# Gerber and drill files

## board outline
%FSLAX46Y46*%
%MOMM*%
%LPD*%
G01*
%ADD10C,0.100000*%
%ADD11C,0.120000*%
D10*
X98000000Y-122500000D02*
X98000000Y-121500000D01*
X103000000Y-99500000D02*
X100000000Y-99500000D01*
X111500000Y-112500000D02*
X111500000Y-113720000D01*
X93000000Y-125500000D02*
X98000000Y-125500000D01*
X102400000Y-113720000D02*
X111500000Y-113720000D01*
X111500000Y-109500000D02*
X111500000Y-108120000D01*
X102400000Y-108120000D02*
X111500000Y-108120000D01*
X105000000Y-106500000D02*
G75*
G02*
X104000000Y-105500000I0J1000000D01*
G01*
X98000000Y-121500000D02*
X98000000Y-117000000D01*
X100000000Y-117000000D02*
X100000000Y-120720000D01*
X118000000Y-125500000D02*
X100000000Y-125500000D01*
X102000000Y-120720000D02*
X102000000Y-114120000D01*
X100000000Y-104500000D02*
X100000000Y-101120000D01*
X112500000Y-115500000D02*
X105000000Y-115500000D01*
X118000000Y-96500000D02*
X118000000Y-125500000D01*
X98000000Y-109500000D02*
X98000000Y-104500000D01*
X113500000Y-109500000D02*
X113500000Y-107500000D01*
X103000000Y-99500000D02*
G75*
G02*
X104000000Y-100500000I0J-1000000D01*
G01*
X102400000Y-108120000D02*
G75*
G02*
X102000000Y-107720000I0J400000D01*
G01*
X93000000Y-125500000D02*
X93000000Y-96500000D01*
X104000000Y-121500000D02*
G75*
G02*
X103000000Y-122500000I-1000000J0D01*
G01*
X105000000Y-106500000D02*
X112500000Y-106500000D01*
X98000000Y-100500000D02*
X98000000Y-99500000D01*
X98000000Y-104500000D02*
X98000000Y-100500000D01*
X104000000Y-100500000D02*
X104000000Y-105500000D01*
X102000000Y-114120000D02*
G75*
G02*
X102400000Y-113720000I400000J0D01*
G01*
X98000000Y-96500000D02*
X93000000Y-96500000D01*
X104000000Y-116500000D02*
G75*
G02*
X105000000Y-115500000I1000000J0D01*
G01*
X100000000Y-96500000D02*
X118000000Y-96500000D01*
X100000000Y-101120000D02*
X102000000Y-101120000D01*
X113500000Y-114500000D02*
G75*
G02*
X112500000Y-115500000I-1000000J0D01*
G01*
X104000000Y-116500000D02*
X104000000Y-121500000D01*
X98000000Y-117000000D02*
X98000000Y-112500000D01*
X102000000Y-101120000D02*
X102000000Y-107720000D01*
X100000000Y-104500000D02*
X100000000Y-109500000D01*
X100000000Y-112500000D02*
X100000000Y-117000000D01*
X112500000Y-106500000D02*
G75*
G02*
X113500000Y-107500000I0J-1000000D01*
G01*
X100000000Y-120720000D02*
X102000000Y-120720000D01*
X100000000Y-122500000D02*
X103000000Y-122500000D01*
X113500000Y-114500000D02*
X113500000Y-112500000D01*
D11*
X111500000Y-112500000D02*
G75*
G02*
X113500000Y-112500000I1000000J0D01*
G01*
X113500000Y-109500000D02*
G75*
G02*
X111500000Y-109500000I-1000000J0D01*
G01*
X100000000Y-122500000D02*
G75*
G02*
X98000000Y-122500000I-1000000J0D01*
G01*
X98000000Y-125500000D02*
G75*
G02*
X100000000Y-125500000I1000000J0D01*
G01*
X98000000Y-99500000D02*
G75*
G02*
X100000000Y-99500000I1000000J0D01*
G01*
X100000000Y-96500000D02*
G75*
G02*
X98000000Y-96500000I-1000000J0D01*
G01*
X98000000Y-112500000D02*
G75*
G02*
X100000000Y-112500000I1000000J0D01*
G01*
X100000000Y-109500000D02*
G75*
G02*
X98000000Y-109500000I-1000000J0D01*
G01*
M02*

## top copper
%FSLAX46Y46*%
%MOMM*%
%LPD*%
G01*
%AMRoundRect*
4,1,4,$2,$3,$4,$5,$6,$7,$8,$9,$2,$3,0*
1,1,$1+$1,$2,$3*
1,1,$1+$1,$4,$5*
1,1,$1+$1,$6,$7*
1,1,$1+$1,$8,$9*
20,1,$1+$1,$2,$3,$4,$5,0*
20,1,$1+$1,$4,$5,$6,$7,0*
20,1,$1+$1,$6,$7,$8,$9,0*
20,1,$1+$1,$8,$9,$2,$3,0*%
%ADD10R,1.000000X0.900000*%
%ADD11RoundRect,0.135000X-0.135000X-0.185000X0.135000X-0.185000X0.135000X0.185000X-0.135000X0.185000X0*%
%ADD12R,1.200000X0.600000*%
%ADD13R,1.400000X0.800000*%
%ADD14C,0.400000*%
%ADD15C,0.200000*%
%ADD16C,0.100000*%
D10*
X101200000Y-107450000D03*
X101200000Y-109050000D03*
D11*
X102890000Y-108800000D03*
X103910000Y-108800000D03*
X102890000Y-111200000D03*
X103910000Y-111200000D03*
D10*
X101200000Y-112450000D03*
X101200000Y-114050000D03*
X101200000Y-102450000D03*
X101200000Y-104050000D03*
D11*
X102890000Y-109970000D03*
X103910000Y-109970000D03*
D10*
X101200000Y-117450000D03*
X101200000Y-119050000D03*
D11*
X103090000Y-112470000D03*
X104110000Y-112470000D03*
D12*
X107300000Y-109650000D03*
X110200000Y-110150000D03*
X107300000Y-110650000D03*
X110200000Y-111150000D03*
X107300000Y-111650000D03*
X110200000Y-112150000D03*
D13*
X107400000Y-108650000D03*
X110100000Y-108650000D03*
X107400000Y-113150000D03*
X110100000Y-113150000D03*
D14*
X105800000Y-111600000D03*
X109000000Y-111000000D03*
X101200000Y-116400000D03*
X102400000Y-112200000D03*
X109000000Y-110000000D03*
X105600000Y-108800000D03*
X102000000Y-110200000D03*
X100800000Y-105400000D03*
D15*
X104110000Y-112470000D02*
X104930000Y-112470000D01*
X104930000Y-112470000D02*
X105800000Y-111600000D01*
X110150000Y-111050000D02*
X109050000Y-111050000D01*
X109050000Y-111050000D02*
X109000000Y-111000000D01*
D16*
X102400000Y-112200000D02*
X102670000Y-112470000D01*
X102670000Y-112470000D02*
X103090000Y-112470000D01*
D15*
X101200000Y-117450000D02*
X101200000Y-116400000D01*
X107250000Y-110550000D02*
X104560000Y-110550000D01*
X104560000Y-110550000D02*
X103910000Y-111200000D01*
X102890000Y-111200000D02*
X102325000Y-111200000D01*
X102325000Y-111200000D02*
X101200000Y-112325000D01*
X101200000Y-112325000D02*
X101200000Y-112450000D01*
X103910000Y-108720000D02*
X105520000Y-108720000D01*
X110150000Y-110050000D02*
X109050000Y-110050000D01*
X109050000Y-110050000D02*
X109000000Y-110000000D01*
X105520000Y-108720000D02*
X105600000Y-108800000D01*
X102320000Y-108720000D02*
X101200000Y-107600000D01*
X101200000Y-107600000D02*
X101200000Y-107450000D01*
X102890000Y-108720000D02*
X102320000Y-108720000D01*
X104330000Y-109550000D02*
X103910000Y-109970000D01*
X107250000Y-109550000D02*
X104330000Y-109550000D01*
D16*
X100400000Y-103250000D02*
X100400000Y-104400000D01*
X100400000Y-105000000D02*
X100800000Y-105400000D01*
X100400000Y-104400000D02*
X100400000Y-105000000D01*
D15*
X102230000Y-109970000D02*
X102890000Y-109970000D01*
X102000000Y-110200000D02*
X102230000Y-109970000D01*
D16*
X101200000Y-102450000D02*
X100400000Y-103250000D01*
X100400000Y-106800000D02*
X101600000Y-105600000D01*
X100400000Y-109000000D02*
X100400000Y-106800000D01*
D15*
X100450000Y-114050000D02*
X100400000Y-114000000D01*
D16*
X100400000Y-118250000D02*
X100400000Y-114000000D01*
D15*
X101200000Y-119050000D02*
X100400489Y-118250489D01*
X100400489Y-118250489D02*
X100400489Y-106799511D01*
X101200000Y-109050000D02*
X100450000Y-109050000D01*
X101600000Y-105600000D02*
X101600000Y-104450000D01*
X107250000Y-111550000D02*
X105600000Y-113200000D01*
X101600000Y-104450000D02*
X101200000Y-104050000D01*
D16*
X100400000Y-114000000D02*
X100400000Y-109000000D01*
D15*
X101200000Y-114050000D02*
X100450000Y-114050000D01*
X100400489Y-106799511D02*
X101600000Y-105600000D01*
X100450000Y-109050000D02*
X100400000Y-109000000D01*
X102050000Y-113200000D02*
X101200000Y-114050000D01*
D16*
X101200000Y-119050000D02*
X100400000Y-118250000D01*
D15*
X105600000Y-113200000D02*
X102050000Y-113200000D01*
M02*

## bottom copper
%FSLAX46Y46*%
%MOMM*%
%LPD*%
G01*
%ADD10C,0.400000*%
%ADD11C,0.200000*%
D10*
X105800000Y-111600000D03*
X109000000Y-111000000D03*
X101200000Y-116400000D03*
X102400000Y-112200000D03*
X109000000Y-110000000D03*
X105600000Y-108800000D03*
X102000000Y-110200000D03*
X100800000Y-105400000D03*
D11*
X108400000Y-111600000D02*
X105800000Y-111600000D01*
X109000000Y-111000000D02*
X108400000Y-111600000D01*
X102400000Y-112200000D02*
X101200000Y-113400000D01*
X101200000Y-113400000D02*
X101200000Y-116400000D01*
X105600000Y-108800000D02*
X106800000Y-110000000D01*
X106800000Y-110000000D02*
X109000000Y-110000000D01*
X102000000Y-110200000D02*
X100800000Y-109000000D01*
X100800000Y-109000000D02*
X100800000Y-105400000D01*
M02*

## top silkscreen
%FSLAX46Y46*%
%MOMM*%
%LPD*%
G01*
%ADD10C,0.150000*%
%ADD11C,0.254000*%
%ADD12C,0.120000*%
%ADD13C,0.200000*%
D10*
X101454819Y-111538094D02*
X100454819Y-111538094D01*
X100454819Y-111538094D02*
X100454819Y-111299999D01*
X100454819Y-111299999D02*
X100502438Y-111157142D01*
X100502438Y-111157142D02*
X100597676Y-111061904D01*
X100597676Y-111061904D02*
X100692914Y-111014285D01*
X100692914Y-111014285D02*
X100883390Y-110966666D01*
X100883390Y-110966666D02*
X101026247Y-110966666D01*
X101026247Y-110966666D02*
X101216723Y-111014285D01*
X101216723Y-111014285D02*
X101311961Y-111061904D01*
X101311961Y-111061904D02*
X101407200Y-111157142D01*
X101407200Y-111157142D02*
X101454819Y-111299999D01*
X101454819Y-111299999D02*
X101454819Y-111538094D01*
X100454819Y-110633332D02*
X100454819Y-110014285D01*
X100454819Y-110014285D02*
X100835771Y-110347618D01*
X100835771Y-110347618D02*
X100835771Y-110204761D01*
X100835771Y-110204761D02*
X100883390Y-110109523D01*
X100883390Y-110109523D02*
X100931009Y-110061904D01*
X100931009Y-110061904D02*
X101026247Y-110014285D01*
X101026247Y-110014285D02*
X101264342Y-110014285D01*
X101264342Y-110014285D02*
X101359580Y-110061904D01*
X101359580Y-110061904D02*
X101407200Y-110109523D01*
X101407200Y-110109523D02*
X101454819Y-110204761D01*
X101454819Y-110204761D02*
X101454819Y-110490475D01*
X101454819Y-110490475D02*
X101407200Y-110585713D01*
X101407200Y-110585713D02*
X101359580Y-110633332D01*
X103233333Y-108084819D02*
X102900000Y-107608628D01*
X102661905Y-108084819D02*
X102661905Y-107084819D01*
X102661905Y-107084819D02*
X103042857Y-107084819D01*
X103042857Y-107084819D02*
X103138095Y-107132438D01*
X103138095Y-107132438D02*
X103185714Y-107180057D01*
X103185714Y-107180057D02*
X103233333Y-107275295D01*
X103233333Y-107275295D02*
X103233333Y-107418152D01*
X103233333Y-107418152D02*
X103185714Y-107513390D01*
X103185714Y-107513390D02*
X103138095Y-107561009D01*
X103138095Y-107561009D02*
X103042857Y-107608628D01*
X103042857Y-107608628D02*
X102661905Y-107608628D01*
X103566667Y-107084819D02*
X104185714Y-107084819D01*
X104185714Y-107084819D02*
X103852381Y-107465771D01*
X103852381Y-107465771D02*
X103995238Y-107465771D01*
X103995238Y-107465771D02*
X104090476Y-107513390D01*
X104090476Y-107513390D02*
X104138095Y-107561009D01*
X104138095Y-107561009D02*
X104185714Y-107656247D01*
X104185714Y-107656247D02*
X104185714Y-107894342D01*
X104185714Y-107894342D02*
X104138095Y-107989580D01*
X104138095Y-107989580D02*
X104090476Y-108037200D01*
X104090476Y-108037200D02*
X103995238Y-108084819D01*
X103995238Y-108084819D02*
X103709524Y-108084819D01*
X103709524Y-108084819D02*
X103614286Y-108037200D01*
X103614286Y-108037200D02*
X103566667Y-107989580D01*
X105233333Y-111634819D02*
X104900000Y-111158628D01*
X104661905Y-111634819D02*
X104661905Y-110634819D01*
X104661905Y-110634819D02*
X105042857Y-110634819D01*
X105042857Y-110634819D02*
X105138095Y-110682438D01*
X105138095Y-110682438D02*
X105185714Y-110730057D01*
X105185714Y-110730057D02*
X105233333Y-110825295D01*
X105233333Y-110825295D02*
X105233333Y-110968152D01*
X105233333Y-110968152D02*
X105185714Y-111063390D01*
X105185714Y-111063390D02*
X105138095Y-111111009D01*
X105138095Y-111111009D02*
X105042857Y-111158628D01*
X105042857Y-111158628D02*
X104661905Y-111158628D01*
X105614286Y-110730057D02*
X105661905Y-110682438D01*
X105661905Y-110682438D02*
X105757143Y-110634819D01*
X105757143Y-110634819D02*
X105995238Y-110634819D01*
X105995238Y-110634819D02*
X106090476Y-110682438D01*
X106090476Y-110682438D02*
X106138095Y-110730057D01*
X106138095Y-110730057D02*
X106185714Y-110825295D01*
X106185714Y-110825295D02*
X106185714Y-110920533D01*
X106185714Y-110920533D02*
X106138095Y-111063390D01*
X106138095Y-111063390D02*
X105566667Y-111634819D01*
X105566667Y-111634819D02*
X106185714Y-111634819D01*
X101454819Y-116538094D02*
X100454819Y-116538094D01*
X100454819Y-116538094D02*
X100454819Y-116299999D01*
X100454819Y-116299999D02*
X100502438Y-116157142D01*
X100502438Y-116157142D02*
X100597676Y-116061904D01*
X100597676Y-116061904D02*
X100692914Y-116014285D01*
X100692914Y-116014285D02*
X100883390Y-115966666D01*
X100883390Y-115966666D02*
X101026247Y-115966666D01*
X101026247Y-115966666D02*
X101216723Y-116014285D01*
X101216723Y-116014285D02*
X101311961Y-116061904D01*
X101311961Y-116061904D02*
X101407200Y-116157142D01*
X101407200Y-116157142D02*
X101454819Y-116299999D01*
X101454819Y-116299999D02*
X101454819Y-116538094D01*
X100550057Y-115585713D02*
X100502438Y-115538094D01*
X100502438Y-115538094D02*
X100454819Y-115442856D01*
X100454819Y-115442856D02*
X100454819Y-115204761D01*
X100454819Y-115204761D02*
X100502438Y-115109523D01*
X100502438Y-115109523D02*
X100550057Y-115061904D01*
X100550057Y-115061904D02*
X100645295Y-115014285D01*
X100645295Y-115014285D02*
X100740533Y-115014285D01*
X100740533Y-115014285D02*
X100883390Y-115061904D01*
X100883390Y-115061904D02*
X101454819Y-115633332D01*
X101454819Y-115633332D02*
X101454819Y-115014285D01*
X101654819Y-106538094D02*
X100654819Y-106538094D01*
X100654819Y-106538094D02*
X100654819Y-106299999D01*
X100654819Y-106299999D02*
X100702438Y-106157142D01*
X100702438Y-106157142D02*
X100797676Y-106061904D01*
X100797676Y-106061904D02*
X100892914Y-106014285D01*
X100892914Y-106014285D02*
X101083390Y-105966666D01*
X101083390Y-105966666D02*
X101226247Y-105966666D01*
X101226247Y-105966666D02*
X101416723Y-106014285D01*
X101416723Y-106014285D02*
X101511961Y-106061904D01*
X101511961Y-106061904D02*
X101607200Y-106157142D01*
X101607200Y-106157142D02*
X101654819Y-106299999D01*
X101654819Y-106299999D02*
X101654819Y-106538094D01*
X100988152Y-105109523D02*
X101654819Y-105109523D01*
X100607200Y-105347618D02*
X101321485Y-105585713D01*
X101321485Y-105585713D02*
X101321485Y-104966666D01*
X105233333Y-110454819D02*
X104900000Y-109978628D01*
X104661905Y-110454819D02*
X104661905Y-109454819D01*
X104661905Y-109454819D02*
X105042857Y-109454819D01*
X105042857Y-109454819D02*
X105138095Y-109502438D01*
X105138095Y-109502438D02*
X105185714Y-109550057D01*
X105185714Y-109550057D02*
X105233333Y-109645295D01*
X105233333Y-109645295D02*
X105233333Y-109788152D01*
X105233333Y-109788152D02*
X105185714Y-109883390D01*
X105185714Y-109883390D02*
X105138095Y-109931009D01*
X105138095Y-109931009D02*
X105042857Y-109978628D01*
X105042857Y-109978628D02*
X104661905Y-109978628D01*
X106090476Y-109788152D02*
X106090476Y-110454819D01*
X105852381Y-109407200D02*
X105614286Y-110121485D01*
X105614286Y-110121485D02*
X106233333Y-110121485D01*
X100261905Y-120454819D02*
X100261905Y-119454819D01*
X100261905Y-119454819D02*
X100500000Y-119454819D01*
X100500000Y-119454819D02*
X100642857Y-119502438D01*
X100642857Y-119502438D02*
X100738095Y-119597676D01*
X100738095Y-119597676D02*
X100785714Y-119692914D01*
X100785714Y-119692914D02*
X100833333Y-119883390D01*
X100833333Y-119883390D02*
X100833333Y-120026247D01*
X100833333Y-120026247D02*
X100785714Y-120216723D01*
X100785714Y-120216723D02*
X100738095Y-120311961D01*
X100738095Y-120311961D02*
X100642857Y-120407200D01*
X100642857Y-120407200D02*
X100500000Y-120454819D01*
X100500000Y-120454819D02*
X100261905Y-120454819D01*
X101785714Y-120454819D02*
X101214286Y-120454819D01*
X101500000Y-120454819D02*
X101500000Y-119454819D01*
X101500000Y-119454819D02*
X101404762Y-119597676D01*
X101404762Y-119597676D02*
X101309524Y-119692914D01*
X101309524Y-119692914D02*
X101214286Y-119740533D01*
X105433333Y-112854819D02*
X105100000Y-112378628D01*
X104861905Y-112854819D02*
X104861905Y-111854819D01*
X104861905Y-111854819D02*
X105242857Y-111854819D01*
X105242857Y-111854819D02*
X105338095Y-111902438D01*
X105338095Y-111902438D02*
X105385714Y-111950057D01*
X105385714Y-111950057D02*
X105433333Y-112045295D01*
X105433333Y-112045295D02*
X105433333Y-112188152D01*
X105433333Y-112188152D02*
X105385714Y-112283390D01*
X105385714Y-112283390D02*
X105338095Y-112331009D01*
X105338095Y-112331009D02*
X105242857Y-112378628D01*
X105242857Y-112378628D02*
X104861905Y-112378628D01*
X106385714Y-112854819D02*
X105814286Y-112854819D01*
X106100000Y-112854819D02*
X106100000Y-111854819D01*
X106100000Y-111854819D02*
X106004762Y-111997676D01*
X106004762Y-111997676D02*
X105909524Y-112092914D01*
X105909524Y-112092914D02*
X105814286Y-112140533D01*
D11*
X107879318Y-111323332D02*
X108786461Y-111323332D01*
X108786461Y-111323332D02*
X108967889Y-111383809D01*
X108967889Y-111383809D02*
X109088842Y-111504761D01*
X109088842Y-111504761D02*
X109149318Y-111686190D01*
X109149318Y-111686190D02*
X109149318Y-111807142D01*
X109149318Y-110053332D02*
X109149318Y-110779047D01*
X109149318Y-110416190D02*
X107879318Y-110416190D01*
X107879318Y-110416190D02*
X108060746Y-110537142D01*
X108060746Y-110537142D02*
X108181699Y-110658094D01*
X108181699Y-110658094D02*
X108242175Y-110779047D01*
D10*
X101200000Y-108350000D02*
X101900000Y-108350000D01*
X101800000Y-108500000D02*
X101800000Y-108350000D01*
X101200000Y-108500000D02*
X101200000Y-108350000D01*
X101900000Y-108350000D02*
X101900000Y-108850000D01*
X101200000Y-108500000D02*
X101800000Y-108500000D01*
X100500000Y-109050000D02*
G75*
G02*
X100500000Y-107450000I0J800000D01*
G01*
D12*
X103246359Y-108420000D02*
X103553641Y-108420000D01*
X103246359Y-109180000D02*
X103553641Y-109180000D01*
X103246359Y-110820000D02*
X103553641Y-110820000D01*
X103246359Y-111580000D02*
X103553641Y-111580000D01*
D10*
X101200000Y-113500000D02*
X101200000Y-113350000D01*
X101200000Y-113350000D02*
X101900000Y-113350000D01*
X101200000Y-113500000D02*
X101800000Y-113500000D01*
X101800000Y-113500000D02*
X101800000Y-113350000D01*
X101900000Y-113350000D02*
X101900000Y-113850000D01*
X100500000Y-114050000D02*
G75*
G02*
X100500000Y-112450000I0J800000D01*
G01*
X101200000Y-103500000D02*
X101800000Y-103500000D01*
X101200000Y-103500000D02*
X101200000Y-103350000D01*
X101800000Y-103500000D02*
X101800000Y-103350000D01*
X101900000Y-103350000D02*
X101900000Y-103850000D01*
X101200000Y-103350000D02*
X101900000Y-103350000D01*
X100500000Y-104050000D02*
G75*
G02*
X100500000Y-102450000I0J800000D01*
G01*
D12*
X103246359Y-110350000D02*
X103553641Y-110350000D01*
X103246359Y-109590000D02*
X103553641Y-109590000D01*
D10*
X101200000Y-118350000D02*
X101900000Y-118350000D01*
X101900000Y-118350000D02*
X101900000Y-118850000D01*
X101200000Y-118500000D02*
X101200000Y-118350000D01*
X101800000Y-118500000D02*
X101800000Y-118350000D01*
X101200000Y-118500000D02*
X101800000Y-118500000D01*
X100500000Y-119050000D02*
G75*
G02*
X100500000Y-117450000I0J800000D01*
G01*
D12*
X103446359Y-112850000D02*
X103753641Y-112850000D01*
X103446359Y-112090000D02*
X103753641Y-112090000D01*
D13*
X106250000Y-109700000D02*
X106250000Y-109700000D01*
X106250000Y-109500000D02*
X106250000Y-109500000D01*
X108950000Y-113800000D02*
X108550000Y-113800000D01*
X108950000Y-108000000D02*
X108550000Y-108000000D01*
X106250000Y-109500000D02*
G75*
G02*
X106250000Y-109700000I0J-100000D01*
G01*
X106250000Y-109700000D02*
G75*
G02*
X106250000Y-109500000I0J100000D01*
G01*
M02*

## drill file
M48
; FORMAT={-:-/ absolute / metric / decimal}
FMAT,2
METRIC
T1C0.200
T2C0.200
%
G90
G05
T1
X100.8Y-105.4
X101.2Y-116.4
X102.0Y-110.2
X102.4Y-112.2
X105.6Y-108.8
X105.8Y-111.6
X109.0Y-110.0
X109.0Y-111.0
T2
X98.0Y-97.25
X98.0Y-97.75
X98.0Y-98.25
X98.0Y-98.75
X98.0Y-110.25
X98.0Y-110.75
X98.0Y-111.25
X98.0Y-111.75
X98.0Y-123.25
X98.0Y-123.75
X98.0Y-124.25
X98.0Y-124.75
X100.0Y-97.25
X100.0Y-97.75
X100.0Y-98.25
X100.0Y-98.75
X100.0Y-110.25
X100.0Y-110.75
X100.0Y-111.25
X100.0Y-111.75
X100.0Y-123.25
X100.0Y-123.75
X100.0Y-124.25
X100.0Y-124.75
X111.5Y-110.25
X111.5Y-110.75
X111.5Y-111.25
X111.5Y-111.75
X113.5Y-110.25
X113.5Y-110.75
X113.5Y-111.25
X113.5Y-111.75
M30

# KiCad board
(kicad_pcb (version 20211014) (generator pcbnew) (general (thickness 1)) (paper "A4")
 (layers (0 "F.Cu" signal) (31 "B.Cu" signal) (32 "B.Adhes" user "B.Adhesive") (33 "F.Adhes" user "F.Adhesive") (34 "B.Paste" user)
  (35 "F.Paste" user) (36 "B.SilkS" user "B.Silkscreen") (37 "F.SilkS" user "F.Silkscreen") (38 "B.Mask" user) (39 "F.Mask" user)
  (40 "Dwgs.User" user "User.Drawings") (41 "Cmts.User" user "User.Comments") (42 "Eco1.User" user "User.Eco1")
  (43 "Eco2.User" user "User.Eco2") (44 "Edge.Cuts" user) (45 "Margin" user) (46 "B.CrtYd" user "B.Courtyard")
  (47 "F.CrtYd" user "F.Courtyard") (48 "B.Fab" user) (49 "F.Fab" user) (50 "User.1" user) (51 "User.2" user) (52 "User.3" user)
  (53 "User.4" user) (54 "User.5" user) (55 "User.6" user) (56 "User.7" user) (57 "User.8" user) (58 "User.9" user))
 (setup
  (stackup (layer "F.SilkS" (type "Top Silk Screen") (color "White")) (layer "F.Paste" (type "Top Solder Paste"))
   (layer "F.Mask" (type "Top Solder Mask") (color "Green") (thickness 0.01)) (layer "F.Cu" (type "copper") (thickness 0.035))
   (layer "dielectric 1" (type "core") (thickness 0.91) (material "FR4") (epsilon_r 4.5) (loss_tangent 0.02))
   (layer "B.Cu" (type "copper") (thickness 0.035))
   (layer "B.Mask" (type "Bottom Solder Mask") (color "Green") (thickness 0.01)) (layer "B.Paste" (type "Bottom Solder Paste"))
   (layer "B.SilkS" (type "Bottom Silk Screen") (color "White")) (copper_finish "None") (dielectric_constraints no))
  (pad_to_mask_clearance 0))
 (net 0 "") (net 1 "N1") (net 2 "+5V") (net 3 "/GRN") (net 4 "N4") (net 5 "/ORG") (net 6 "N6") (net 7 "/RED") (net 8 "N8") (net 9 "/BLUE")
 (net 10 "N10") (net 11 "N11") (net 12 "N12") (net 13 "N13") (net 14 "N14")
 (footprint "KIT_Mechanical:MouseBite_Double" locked (layer "F.Cu") (at 112.5 111) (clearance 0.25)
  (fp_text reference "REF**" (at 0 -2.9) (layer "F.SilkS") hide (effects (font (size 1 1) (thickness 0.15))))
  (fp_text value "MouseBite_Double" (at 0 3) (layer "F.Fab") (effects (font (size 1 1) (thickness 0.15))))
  (fp_arc (start -1 1.5) (mid 0 0.5) (end 1 1.5) (layer "Edge.Cuts") (width 0.12))
  (fp_arc (start 1 -1.5) (mid 0 -0.5) (end -1 -1.5) (layer "Edge.Cuts") (width 0.12))
  (pad "" np_thru_hole circle locked (at -1 0.75) (size 0.2 0.2) (drill 0.2) (layers *.Cu *.Mask))
  (pad "" np_thru_hole circle locked (at -1 0.25) (size 0.2 0.2) (drill 0.2) (layers *.Cu *.Mask))
  (pad "" np_thru_hole circle locked (at -1 -0.25) (size 0.2 0.2) (drill 0.2) (layers *.Cu *.Mask))
  (pad "" np_thru_hole circle locked (at -1 -0.75) (size 0.2 0.2) (drill 0.2) (layers *.Cu *.Mask))
  (pad "" np_thru_hole circle locked (at 1 0.75 180) (size 0.2 0.2) (drill 0.2) (layers *.Cu *.Mask))
  (pad "" np_thru_hole circle locked (at 1 -0.25 180) (size 0.2 0.2) (drill 0.2) (layers *.Cu *.Mask))
  (pad "" np_thru_hole circle locked (at 1 0.25 180) (size 0.2 0.2) (drill 0.2) (layers *.Cu *.Mask))
  (pad "" np_thru_hole circle locked (at 1 -0.75 180) (size 0.2 0.2) (drill 0.2) (layers *.Cu *.Mask)))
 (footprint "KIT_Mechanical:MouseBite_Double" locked (layer "F.Cu") (at 99 124) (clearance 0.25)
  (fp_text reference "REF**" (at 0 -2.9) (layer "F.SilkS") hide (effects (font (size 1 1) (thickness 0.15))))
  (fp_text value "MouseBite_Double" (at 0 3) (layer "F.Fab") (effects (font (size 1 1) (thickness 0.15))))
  (fp_arc (start 1 -1.5) (mid 0 -0.5) (end -1 -1.5) (layer "Edge.Cuts") (width 0.12))
  (fp_arc (start -1 1.5) (mid 0 0.5) (end 1 1.5) (layer "Edge.Cuts") (width 0.12))
  (pad "" np_thru_hole circle locked (at -1 -0.75) (size 0.2 0.2) (drill 0.2) (layers *.Cu *.Mask))
  (pad "" np_thru_hole circle locked (at -1 0.25) (size 0.2 0.2) (drill 0.2) (layers *.Cu *.Mask))
  (pad "" np_thru_hole circle locked (at 1 0.25 180) (size 0.2 0.2) (drill 0.2) (layers *.Cu *.Mask))
  (pad "" np_thru_hole circle locked (at 1 -0.75 180) (size 0.2 0.2) (drill 0.2) (layers *.Cu *.Mask))
  (pad "" np_thru_hole circle locked (at -1 -0.25) (size 0.2 0.2) (drill 0.2) (layers *.Cu *.Mask))
  (pad "" np_thru_hole circle locked (at -1 0.75) (size 0.2 0.2) (drill 0.2) (layers *.Cu *.Mask))
  (pad "" np_thru_hole circle locked (at 1 0.75 180) (size 0.2 0.2) (drill 0.2) (layers *.Cu *.Mask))
  (pad "" np_thru_hole circle locked (at 1 -0.25 180) (size 0.2 0.2) (drill 0.2) (layers *.Cu *.Mask)))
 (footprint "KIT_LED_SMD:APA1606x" (layer "F.Cu") (at 101.2 108.25 -90)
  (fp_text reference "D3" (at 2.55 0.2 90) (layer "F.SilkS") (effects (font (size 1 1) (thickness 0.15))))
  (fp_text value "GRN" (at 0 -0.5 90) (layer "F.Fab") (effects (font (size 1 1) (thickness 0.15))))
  (fp_line (start 0.1 0) (end 0.1 -0.7) (layer "F.SilkS") (width 0.15))
  (fp_line (start 0.25 -0.6) (end 0.1 -0.6) (layer "F.SilkS") (width 0.15))
  (fp_line (start 0.25 0) (end 0.1 0) (layer "F.SilkS") (width 0.15))
  (fp_line (start 0.1 -0.7) (end 0.6 -0.7) (layer "F.SilkS") (width 0.15))
  (fp_line (start 0.25 0) (end 0.25 -0.6) (layer "F.SilkS") (width 0.15))
  (fp_arc (start 0.8 0.7) (mid 0 1.5) (end -0.8 0.7) (layer "F.SilkS") (width 0.15))
  (pad "1" smd rect (at -0.8 0 270) (size 0.9 1) (layers "F.Cu" "F.Paste" "F.Mask") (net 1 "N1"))
  (pad "2" smd rect (at 0.8 0 270) (size 0.9 1) (layers "F.Cu" "F.Paste" "F.Mask") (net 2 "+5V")))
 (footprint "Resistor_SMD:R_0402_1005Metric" (layer "F.Cu") (at 103.4 108.8)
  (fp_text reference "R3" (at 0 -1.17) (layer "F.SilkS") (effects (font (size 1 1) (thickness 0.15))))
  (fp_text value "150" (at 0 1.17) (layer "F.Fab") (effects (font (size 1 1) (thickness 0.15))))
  (fp_line (start -0.153641 -0.38) (end 0.153641 -0.38) (layer "F.SilkS") (width 0.12))
  (fp_line (start -0.153641 0.38) (end 0.153641 0.38) (layer "F.SilkS") (width 0.12))
  (pad "1" smd roundrect (at -0.51 0) (size 0.54 0.64) (layers "F.Cu" "F.Paste" "F.Mask") (roundrect_rratio 0.25) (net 1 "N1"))
  (pad "2" smd roundrect (at 0.51 0) (size 0.54 0.64) (layers "F.Cu" "F.Paste" "F.Mask") (roundrect_rratio 0.25) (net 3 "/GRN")))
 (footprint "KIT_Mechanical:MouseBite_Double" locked (layer "F.Cu") (at 99 98) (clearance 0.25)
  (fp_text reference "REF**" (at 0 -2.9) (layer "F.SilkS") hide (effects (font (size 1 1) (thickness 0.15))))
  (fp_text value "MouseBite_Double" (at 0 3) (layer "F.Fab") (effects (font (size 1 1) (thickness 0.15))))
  (fp_arc (start -1 1.5) (mid 0 0.5) (end 1 1.5) (layer "Edge.Cuts") (width 0.12))
  (fp_arc (start 1 -1.5) (mid 0 -0.5) (end -1 -1.5) (layer "Edge.Cuts") (width 0.12))
  (pad "" np_thru_hole circle locked (at 1 -0.75 180) (size 0.2 0.2) (drill 0.2) (layers *.Cu *.Mask))
  (pad "" np_thru_hole circle locked (at -1 -0.75) (size 0.2 0.2) (drill 0.2) (layers *.Cu *.Mask))
  (pad "" np_thru_hole circle locked (at 1 -0.25 180) (size 0.2 0.2) (drill 0.2) (layers *.Cu *.Mask))
  (pad "" np_thru_hole circle locked (at -1 0.25) (size 0.2 0.2) (drill 0.2) (layers *.Cu *.Mask))
  (pad "" np_thru_hole circle locked (at 1 0.25 180) (size 0.2 0.2) (drill 0.2) (layers *.Cu *.Mask))
  (pad "" np_thru_hole circle locked (at -1 0.75) (size 0.2 0.2) (drill 0.2) (layers *.Cu *.Mask))
  (pad "" np_thru_hole circle locked (at -1 -0.25) (size 0.2 0.2) (drill 0.2) (layers *.Cu *.Mask))
  (pad "" np_thru_hole circle locked (at 1 0.75 180) (size 0.2 0.2) (drill 0.2) (layers *.Cu *.Mask)))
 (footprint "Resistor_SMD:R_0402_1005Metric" (layer "F.Cu") (at 103.4 111.2)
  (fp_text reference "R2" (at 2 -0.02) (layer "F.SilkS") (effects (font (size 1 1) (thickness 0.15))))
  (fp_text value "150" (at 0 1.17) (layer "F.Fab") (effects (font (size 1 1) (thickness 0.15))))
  (fp_line (start -0.153641 -0.38) (end 0.153641 -0.38) (layer "F.SilkS") (width 0.12))
  (fp_line (start -0.153641 0.38) (end 0.153641 0.38) (layer "F.SilkS") (width 0.12))
  (pad "1" smd roundrect (at -0.51 0) (size 0.54 0.64) (layers "F.Cu" "F.Paste" "F.Mask") (roundrect_rratio 0.25) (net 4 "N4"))
  (pad "2" smd roundrect (at 0.51 0) (size 0.54 0.64) (layers "F.Cu" "F.Paste" "F.Mask") (roundrect_rratio 0.25) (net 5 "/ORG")))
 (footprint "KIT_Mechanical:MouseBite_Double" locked (layer "F.Cu") (at 99 111) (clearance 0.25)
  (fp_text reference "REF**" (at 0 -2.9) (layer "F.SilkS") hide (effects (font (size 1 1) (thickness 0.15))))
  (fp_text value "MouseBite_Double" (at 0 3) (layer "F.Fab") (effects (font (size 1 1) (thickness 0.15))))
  (fp_arc (start -1 1.5) (mid 0 0.5) (end 1 1.5) (layer "Edge.Cuts") (width 0.12))
  (fp_arc (start 1 -1.5) (mid 0 -0.5) (end -1 -1.5) (layer "Edge.Cuts") (width 0.12))
  (pad "" np_thru_hole circle locked (at -1 -0.25) (size 0.2 0.2) (drill 0.2) (layers *.Cu *.Mask))
  (pad "" np_thru_hole circle locked (at -1 -0.75) (size 0.2 0.2) (drill 0.2) (layers *.Cu *.Mask))
  (pad "" np_thru_hole circle locked (at -1 0.25) (size 0.2 0.2) (drill 0.2) (layers *.Cu *.Mask))
  (pad "" np_thru_hole circle locked (at 1 0.25 180) (size 0.2 0.2) (drill 0.2) (layers *.Cu *.Mask))
  (pad "" np_thru_hole circle locked (at 1 -0.75 180) (size 0.2 0.2) (drill 0.2) (layers *.Cu *.Mask))
  (pad "" np_thru_hole circle locked (at 1 0.75 180) (size 0.2 0.2) (drill 0.2) (layers *.Cu *.Mask))
  (pad "" np_thru_hole circle locked (at 1 -0.25 180) (size 0.2 0.2) (drill 0.2) (layers *.Cu *.Mask))
  (pad "" np_thru_hole circle locked (at -1 0.75) (size 0.2 0.2) (drill 0.2) (layers *.Cu *.Mask)))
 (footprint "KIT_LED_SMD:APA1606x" (layer "F.Cu") (at 101.2 113.25 -90)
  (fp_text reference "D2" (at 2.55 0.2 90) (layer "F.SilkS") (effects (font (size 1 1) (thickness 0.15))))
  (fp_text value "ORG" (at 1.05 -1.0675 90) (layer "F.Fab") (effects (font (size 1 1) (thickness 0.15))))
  (fp_line (start 0.25 0) (end 0.1 0) (layer "F.SilkS") (width 0.15))
  (fp_line (start 0.1 0) (end 0.1 -0.7) (layer "F.SilkS") (width 0.15))
  (fp_line (start 0.25 0) (end 0.25 -0.6) (layer "F.SilkS") (width 0.15))
  (fp_line (start 0.25 -0.6) (end 0.1 -0.6) (layer "F.SilkS") (width 0.15))
  (fp_line (start 0.1 -0.7) (end 0.6 -0.7) (layer "F.SilkS") (width 0.15))
  (fp_arc (start 0.8 0.7) (mid 0 1.5) (end -0.8 0.7) (layer "F.SilkS") (width 0.15))
  (pad "1" smd rect (at -0.8 0 270) (size 0.9 1) (layers "F.Cu" "F.Paste" "F.Mask") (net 4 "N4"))
  (pad "2" smd rect (at 0.8 0 270) (size 0.9 1) (layers "F.Cu" "F.Paste" "F.Mask") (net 2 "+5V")))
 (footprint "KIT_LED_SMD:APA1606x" (layer "F.Cu") (at 101.2 103.25 -90)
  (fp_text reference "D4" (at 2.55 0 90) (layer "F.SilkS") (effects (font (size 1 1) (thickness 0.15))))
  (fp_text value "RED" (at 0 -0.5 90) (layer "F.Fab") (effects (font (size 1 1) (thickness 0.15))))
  (fp_line (start 0.25 0) (end 0.25 -0.6) (layer "F.SilkS") (width 0.15))
  (fp_line (start 0.25 0) (end 0.1 0) (layer "F.SilkS") (width 0.15))
  (fp_line (start 0.25 -0.6) (end 0.1 -0.6) (layer "F.SilkS") (width 0.15))
  (fp_line (start 0.1 -0.7) (end 0.6 -0.7) (layer "F.SilkS") (width 0.15))
  (fp_line (start 0.1 0) (end 0.1 -0.7) (layer "F.SilkS") (width 0.15))
  (fp_arc (start 0.8 0.7) (mid 0 1.5) (end -0.8 0.7) (layer "F.SilkS") (width 0.15))
  (pad "1" smd rect (at -0.8 0 270) (size 0.9 1) (layers "F.Cu" "F.Paste" "F.Mask") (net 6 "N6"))
  (pad "2" smd rect (at 0.8 0 270) (size 0.9 1) (layers "F.Cu" "F.Paste" "F.Mask") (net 2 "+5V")))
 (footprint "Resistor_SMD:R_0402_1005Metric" (layer "F.Cu") (at 103.4 109.97)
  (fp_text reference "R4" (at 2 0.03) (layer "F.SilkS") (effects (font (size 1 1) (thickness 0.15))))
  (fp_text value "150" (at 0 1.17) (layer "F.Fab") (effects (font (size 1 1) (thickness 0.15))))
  (fp_line (start -0.153641 0.38) (end 0.153641 0.38) (layer "F.SilkS") (width 0.12))
  (fp_line (start -0.153641 -0.38) (end 0.153641 -0.38) (layer "F.SilkS") (width 0.12))
  (pad "1" smd roundrect (at -0.51 0) (size 0.54 0.64) (layers "F.Cu" "F.Paste" "F.Mask") (roundrect_rratio 0.25) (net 6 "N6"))
  (pad "2" smd roundrect (at 0.51 0) (size 0.54 0.64) (layers "F.Cu" "F.Paste" "F.Mask") (roundrect_rratio 0.25) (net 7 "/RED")))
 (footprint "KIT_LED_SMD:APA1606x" (layer "F.Cu") (at 101.2 118.25 -90)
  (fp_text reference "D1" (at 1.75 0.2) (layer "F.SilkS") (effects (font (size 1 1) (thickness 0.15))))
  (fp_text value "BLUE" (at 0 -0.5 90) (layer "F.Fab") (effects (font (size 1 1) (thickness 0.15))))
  (fp_line (start 0.1 0) (end 0.1 -0.7) (layer "F.SilkS") (width 0.15))
  (fp_line (start 0.1 -0.7) (end 0.6 -0.7) (layer "F.SilkS") (width 0.15))
  (fp_line (start 0.25 0) (end 0.1 0) (layer "F.SilkS") (width 0.15))
  (fp_line (start 0.25 -0.6) (end 0.1 -0.6) (layer "F.SilkS") (width 0.15))
  (fp_line (start 0.25 0) (end 0.25 -0.6) (layer "F.SilkS") (width 0.15))
  (fp_arc (start 0.8 0.7) (mid 0 1.5) (end -0.8 0.7) (layer "F.SilkS") (width 0.15))
  (pad "1" smd rect (at -0.8 0 270) (size 0.9 1) (layers "F.Cu" "F.Paste" "F.Mask") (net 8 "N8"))
  (pad "2" smd rect (at 0.8 0 270) (size 0.9 1) (layers "F.Cu" "F.Paste" "F.Mask") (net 2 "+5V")))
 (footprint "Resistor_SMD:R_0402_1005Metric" (layer "F.Cu") (at 103.6 112.47)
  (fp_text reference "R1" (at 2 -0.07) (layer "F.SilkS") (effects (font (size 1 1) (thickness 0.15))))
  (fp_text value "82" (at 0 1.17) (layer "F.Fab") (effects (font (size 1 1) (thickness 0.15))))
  (fp_line (start -0.153641 0.38) (end 0.153641 0.38) (layer "F.SilkS") (width 0.12))
  (fp_line (start -0.153641 -0.38) (end 0.153641 -0.38) (layer "F.SilkS") (width 0.12))
  (pad "1" smd roundrect (at -0.51 0) (size 0.54 0.64) (layers "F.Cu" "F.Paste" "F.Mask") (roundrect_rratio 0.25) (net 8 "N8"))
  (pad "2" smd roundrect (at 0.51 0) (size 0.54 0.64) (layers "F.Cu" "F.Paste" "F.Mask") (roundrect_rratio 0.25) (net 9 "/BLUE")))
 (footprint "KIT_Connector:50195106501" (layer "F.Cu") (at 108.75 110.9 -90)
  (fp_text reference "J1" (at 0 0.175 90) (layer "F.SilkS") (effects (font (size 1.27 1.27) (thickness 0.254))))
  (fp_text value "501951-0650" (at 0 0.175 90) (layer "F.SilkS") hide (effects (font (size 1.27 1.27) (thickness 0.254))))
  (fp_line (start -1.2 2.5) (end -1.2 2.5) (layer "F.SilkS") (width 0.2))
  (fp_line (start -1.4 2.5) (end -1.4 2.5) (layer "F.SilkS") (width 0.2))
  (fp_line (start 2.9 -0.2) (end 2.9 0.2) (layer "F.SilkS") (width 0.2))
  (fp_line (start -2.9 -0.2) (end -2.9 0.2) (layer "F.SilkS") (width 0.2))
  (fp_arc (start -1.4 2.5) (mid -1.3 2.4) (end -1.2 2.5) (layer "F.SilkS") (width 0.2))
  (fp_arc (start -1.2 2.5) (mid -1.3 2.6) (end -1.4 2.5) (layer "F.SilkS") (width 0.2))
  (pad "1" smd rect (at -1.25 1.45 270) (size 0.6 1.2) (layers "F.Cu" "F.Paste" "F.Mask") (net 7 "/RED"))
  (pad "2" smd rect (at -0.75 -1.45 270) (size 0.6 1.2) (layers "F.Cu" "F.Paste" "F.Mask") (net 3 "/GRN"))
  (pad "3" smd rect (at -0.25 1.45 270) (size 0.6 1.2) (layers "F.Cu" "F.Paste" "F.Mask") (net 5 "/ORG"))
  (pad "4" smd rect (at 0.25 -1.45 270) (size 0.6 1.2) (layers "F.Cu" "F.Paste" "F.Mask") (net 9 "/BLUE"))
  (pad "5" smd rect (at 0.75 1.45 270) (size 0.6 1.2) (layers "F.Cu" "F.Paste" "F.Mask") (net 2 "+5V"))
  (pad "6" smd rect (at 1.25 -1.45 270) (size 0.6 1.2) (layers "F.Cu" "F.Paste" "F.Mask") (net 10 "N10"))
  (pad "MP1" smd rect (at -2.25 1.35 270) (size 0.8 1.4) (layers "F.Cu" "F.Paste" "F.Mask") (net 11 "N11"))
  (pad "MP2" smd rect (at -2.25 -1.35 270) (size 0.8 1.4) (layers "F.Cu" "F.Paste" "F.Mask") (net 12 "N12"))
  (pad "MP3" smd rect (at 2.25 1.35 270) (size 0.8 1.4) (layers "F.Cu" "F.Paste" "F.Mask") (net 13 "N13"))
  (pad "MP4" smd rect (at 2.25 -1.35 270) (size 0.8 1.4) (layers "F.Cu" "F.Paste" "F.Mask") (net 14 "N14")))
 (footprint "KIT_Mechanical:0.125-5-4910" (layer "B.Cu") (at 110.7 112.52 180)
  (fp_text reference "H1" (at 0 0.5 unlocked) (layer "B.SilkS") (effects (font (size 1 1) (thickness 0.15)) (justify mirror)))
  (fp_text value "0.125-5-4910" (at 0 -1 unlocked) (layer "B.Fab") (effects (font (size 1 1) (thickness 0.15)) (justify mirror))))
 (gr_line (start 98 122.5) (end 98 121.5) (layer "Edge.Cuts") (width 0.1))
 (gr_line (start 103 99.5) (end 100 99.5) (layer "Edge.Cuts") (width 0.1))
 (gr_line (start 111.5 112.5) (end 111.5 113.72) (layer "Edge.Cuts") (width 0.1))
 (gr_line (start 93 125.5) (end 98 125.5) (layer "Edge.Cuts") (width 0.1))
 (gr_line (start 102.4 113.72) (end 111.5 113.72) (layer "Edge.Cuts") (width 0.1))
 (gr_line (start 111.5 109.5) (end 111.5 108.12) (layer "Edge.Cuts") (width 0.1))
 (gr_line (start 102.4 108.12) (end 111.5 108.12) (layer "Edge.Cuts") (width 0.1))
 (gr_arc (start 105 106.5) (mid 104.292893 106.207107) (end 104 105.5) (layer "Edge.Cuts") (width 0.1))
 (gr_line (start 98 121.5) (end 98 117) (layer "Edge.Cuts") (width 0.1))
 (gr_line (start 100 117) (end 100 120.72) (layer "Edge.Cuts") (width 0.1))
 (gr_line (start 118 125.5) (end 100 125.5) (layer "Edge.Cuts") (width 0.1))
 (gr_line (start 102 120.72) (end 102 114.12) (layer "Edge.Cuts") (width 0.1))
 (gr_line (start 100 104.5) (end 100 101.12) (layer "Edge.Cuts") (width 0.1))
 (gr_line (start 112.5 115.5) (end 105 115.5) (layer "Edge.Cuts") (width 0.1))
 (gr_line (start 118 96.5) (end 118 125.5) (layer "Edge.Cuts") (width 0.1))
 (gr_line (start 98 109.5) (end 98 104.5) (layer "Edge.Cuts") (width 0.1))
 (gr_line (start 113.5 109.5) (end 113.5 107.5) (layer "Edge.Cuts") (width 0.1))
 (gr_arc (start 103 99.5) (mid 103.707107 99.792893) (end 104 100.5) (layer "Edge.Cuts") (width 0.1))
 (gr_arc (start 102.4 108.12) (mid 102.117157 108.002843) (end 102 107.72) (layer "Edge.Cuts") (width 0.1))
 (gr_line (start 93 125.5) (end 93 96.5) (layer "Edge.Cuts") (width 0.1))
 (gr_arc (start 104 121.5) (mid 103.707107 122.207107) (end 103 122.5) (layer "Edge.Cuts") (width 0.1))
 (gr_line (start 105 106.5) (end 112.5 106.5) (layer "Edge.Cuts") (width 0.1))
 (gr_line (start 98 100.5) (end 98 99.5) (layer "Edge.Cuts") (width 0.1))
 (gr_line (start 98 104.5) (end 98 100.5) (layer "Edge.Cuts") (width 0.1))
 (gr_line (start 104 100.5) (end 104 105.5) (layer "Edge.Cuts") (width 0.1))
 (gr_arc (start 102 114.12) (mid 102.117157 113.837157) (end 102.4 113.72) (layer "Edge.Cuts") (width 0.1))
 (gr_line (start 98 96.5) (end 93 96.5) (layer "Edge.Cuts") (width 0.1))
 (gr_arc (start 104 116.5) (mid 104.292893 115.792893) (end 105 115.5) (layer "Edge.Cuts") (width 0.1))
 (gr_line (start 100 96.5) (end 118 96.5) (layer "Edge.Cuts") (width 0.1))
 (gr_line (start 100 101.12) (end 102 101.12) (layer "Edge.Cuts") (width 0.1))
 (gr_arc (start 113.5 114.5) (mid 113.207107 115.207107) (end 112.5 115.5) (layer "Edge.Cuts") (width 0.1))
 (gr_line (start 104 116.5) (end 104 121.5) (layer "Edge.Cuts") (width 0.1))
 (gr_line (start 98 117) (end 98 112.5) (layer "Edge.Cuts") (width 0.1))
 (gr_line (start 102 101.12) (end 102 107.72) (layer "Edge.Cuts") (width 0.1))
 (gr_line (start 100 104.5) (end 100 109.5) (layer "Edge.Cuts") (width 0.1))
 (gr_line (start 100 112.5) (end 100 117) (layer "Edge.Cuts") (width 0.1))
 (gr_arc (start 112.5 106.5) (mid 113.207107 106.792893) (end 113.5 107.5) (layer "Edge.Cuts") (width 0.1))
 (gr_line (start 100 120.72) (end 102 120.72) (layer "Edge.Cuts") (width 0.1))
 (gr_line (start 100 122.5) (end 103 122.5) (layer "Edge.Cuts") (width 0.1))
 (gr_line (start 113.5 114.5) (end 113.5 112.5) (layer "Edge.Cuts") (width 0.1))
 (segment (start 104.11 112.47) (end 104.93 112.47) (width 0.2) (layer "F.Cu") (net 9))
 (segment (start 104.93 112.47) (end 105.8 111.6) (width 0.2) (layer "F.Cu") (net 9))
 (segment (start 110.15 111.05) (end 109.05 111.05) (width 0.2) (layer "F.Cu") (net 9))
 (segment (start 109.05 111.05) (end 109 111) (width 0.2) (layer "F.Cu") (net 9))
 (via (at 105.8 111.6) (size 0.4) (drill 0.2) (layers "F.Cu" "B.Cu") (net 9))
 (via (at 109 111) (size 0.4) (drill 0.2) (layers "F.Cu" "B.Cu") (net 9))
 (segment (start 108.4 111.6) (end 105.8 111.6) (width 0.2) (layer "B.Cu") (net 9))
 (segment (start 109 111) (end 108.4 111.6) (width 0.2) (layer "B.Cu") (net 9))
 (segment (start 102.4 112.2) (end 102.67 112.47) (width 0.1) (layer "F.Cu") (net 8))
 (segment (start 102.67 112.47) (end 103.09 112.47) (width 0.1) (layer "F.Cu") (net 8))
 (segment (start 101.2 117.45) (end 101.2 116.4) (width 0.2) (layer "F.Cu") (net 8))
 (via (at 101.2 116.4) (size 0.4) (drill 0.2) (layers "F.Cu" "B.Cu") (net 8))
 (via (at 102.4 112.2) (size 0.4) (drill 0.2) (layers "F.Cu" "B.Cu") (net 8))
 (segment (start 102.4 112.2) (end 101.2 113.4) (width 0.2) (layer "B.Cu") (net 8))
 (segment (start 101.2 113.4) (end 101.2 116.4) (width 0.2) (layer "B.Cu") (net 8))
 (segment (start 107.25 110.55) (end 104.56 110.55) (width 0.2) (layer "F.Cu") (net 5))
 (segment (start 104.56 110.55) (end 103.91 111.2) (width 0.2) (layer "F.Cu") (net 5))
 (segment (start 102.89 111.2) (end 102.325 111.2) (width 0.2) (layer "F.Cu") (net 4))
 (segment (start 102.325 111.2) (end 101.2 112.325) (width 0.2) (layer "F.Cu") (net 4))
 (segment (start 101.2 112.325) (end 101.2 112.45) (width 0.2) (layer "F.Cu") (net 4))
 (segment (start 103.91 108.72) (end 105.52 108.72) (width 0.2) (layer "F.Cu") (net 3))
 (segment (start 110.15 110.05) (end 109.05 110.05) (width 0.2) (layer "F.Cu") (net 3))
 (segment (start 109.05 110.05) (end 109 110) (width 0.2) (layer "F.Cu") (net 3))
 (segment (start 105.52 108.72) (end 105.6 108.8) (width 0.2) (layer "F.Cu") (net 3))
 (via (at 109 110) (size 0.4) (drill 0.2) (layers "F.Cu" "B.Cu") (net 3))
 (via (at 105.6 108.8) (size 0.4) (drill 0.2) (layers "F.Cu" "B.Cu") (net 3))
 (segment (start 105.6 108.8) (end 106.8 110) (width 0.2) (layer "B.Cu") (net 3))
 (segment (start 106.8 110) (end 109 110) (width 0.2) (layer "B.Cu") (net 3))
 (segment (start 102.32 108.72) (end 101.2 107.6) (width 0.2) (layer "F.Cu") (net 1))
 (segment (start 101.2 107.6) (end 101.2 107.45) (width 0.2) (layer "F.Cu") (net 1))
 (segment (start 102.89 108.72) (end 102.32 108.72) (width 0.2) (layer "F.Cu") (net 1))
 (segment (start 104.33 109.55) (end 103.91 109.97) (width 0.2) (layer "F.Cu") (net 7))
 (segment (start 107.25 109.55) (end 104.33 109.55) (width 0.2) (layer "F.Cu") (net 7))
 (segment (start 100.4 103.25) (end 100.4 104.4) (width 0.1) (layer "F.Cu") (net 6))
 (segment (start 100.4 105) (end 100.8 105.4) (width 0.1) (layer "F.Cu") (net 6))
 (segment (start 100.4 104.4) (end 100.4 105) (width 0.1) (layer "F.Cu") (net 6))
 (segment (start 102.23 109.97) (end 102.89 109.97) (width 0.2) (layer "F.Cu") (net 6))
 (segment (start 102 110.2) (end 102.23 109.97) (width 0.2) (layer "F.Cu") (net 6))
 (segment (start 101.2 102.45) (end 100.4 103.25) (width 0.1) (layer "F.Cu") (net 6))
 (via (at 102 110.2) (size 0.4) (drill 0.2) (layers "F.Cu" "B.Cu") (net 6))
 (via (at 100.8 105.4) (size 0.4) (drill 0.2) (layers "F.Cu" "B.Cu") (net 6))
 (segment (start 102 110.2) (end 100.8 109) (width 0.2) (layer "B.Cu") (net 6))
 (segment (start 100.8 109) (end 100.8 105.4) (width 0.2) (layer "B.Cu") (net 6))
 (segment (start 100.4 106.8) (end 101.6 105.6) (width 0.1) (layer "F.Cu") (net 2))
 (segment (start 100.4 109) (end 100.4 106.8) (width 0.1) (layer "F.Cu") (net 2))
 (segment (start 100.45 114.05) (end 100.4 114) (width 0.2) (layer "F.Cu") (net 2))
 (segment (start 100.4 118.25) (end 100.4 114) (width 0.1) (layer "F.Cu") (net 2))
 (segment (start 101.2 119.05) (end 100.400489 118.250489) (width 0.2) (layer "F.Cu") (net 2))
 (segment (start 100.400489 118.250489) (end 100.400489 106.799511) (width 0.2) (layer "F.Cu") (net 2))
 (segment (start 101.2 109.05) (end 100.45 109.05) (width 0.2) (layer "F.Cu") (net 2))
 (segment (start 101.6 105.6) (end 101.6 104.45) (width 0.2) (layer "F.Cu") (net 2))
 (segment (start 107.25 111.55) (end 105.6 113.2) (width 0.2) (layer "F.Cu") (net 2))
 (segment (start 101.6 104.45) (end 101.2 104.05) (width 0.2) (layer "F.Cu") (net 2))
 (segment (start 100.4 114) (end 100.4 109) (width 0.1) (layer "F.Cu") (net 2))
 (segment (start 101.2 114.05) (end 100.45 114.05) (width 0.2) (layer "F.Cu") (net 2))
 (segment (start 100.400489 106.799511) (end 101.6 105.6) (width 0.2) (layer "F.Cu") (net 2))
 (segment (start 100.45 109.05) (end 100.4 109) (width 0.2) (layer "F.Cu") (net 2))
 (segment (start 102.05 113.2) (end 101.2 114.05) (width 0.2) (layer "F.Cu") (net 2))
 (segment (start 101.2 119.05) (end 100.4 118.25) (width 0.1) (layer "F.Cu") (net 2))
 (segment (start 105.6 113.2) (end 102.05 113.2) (width 0.2) (layer "F.Cu") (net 2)))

